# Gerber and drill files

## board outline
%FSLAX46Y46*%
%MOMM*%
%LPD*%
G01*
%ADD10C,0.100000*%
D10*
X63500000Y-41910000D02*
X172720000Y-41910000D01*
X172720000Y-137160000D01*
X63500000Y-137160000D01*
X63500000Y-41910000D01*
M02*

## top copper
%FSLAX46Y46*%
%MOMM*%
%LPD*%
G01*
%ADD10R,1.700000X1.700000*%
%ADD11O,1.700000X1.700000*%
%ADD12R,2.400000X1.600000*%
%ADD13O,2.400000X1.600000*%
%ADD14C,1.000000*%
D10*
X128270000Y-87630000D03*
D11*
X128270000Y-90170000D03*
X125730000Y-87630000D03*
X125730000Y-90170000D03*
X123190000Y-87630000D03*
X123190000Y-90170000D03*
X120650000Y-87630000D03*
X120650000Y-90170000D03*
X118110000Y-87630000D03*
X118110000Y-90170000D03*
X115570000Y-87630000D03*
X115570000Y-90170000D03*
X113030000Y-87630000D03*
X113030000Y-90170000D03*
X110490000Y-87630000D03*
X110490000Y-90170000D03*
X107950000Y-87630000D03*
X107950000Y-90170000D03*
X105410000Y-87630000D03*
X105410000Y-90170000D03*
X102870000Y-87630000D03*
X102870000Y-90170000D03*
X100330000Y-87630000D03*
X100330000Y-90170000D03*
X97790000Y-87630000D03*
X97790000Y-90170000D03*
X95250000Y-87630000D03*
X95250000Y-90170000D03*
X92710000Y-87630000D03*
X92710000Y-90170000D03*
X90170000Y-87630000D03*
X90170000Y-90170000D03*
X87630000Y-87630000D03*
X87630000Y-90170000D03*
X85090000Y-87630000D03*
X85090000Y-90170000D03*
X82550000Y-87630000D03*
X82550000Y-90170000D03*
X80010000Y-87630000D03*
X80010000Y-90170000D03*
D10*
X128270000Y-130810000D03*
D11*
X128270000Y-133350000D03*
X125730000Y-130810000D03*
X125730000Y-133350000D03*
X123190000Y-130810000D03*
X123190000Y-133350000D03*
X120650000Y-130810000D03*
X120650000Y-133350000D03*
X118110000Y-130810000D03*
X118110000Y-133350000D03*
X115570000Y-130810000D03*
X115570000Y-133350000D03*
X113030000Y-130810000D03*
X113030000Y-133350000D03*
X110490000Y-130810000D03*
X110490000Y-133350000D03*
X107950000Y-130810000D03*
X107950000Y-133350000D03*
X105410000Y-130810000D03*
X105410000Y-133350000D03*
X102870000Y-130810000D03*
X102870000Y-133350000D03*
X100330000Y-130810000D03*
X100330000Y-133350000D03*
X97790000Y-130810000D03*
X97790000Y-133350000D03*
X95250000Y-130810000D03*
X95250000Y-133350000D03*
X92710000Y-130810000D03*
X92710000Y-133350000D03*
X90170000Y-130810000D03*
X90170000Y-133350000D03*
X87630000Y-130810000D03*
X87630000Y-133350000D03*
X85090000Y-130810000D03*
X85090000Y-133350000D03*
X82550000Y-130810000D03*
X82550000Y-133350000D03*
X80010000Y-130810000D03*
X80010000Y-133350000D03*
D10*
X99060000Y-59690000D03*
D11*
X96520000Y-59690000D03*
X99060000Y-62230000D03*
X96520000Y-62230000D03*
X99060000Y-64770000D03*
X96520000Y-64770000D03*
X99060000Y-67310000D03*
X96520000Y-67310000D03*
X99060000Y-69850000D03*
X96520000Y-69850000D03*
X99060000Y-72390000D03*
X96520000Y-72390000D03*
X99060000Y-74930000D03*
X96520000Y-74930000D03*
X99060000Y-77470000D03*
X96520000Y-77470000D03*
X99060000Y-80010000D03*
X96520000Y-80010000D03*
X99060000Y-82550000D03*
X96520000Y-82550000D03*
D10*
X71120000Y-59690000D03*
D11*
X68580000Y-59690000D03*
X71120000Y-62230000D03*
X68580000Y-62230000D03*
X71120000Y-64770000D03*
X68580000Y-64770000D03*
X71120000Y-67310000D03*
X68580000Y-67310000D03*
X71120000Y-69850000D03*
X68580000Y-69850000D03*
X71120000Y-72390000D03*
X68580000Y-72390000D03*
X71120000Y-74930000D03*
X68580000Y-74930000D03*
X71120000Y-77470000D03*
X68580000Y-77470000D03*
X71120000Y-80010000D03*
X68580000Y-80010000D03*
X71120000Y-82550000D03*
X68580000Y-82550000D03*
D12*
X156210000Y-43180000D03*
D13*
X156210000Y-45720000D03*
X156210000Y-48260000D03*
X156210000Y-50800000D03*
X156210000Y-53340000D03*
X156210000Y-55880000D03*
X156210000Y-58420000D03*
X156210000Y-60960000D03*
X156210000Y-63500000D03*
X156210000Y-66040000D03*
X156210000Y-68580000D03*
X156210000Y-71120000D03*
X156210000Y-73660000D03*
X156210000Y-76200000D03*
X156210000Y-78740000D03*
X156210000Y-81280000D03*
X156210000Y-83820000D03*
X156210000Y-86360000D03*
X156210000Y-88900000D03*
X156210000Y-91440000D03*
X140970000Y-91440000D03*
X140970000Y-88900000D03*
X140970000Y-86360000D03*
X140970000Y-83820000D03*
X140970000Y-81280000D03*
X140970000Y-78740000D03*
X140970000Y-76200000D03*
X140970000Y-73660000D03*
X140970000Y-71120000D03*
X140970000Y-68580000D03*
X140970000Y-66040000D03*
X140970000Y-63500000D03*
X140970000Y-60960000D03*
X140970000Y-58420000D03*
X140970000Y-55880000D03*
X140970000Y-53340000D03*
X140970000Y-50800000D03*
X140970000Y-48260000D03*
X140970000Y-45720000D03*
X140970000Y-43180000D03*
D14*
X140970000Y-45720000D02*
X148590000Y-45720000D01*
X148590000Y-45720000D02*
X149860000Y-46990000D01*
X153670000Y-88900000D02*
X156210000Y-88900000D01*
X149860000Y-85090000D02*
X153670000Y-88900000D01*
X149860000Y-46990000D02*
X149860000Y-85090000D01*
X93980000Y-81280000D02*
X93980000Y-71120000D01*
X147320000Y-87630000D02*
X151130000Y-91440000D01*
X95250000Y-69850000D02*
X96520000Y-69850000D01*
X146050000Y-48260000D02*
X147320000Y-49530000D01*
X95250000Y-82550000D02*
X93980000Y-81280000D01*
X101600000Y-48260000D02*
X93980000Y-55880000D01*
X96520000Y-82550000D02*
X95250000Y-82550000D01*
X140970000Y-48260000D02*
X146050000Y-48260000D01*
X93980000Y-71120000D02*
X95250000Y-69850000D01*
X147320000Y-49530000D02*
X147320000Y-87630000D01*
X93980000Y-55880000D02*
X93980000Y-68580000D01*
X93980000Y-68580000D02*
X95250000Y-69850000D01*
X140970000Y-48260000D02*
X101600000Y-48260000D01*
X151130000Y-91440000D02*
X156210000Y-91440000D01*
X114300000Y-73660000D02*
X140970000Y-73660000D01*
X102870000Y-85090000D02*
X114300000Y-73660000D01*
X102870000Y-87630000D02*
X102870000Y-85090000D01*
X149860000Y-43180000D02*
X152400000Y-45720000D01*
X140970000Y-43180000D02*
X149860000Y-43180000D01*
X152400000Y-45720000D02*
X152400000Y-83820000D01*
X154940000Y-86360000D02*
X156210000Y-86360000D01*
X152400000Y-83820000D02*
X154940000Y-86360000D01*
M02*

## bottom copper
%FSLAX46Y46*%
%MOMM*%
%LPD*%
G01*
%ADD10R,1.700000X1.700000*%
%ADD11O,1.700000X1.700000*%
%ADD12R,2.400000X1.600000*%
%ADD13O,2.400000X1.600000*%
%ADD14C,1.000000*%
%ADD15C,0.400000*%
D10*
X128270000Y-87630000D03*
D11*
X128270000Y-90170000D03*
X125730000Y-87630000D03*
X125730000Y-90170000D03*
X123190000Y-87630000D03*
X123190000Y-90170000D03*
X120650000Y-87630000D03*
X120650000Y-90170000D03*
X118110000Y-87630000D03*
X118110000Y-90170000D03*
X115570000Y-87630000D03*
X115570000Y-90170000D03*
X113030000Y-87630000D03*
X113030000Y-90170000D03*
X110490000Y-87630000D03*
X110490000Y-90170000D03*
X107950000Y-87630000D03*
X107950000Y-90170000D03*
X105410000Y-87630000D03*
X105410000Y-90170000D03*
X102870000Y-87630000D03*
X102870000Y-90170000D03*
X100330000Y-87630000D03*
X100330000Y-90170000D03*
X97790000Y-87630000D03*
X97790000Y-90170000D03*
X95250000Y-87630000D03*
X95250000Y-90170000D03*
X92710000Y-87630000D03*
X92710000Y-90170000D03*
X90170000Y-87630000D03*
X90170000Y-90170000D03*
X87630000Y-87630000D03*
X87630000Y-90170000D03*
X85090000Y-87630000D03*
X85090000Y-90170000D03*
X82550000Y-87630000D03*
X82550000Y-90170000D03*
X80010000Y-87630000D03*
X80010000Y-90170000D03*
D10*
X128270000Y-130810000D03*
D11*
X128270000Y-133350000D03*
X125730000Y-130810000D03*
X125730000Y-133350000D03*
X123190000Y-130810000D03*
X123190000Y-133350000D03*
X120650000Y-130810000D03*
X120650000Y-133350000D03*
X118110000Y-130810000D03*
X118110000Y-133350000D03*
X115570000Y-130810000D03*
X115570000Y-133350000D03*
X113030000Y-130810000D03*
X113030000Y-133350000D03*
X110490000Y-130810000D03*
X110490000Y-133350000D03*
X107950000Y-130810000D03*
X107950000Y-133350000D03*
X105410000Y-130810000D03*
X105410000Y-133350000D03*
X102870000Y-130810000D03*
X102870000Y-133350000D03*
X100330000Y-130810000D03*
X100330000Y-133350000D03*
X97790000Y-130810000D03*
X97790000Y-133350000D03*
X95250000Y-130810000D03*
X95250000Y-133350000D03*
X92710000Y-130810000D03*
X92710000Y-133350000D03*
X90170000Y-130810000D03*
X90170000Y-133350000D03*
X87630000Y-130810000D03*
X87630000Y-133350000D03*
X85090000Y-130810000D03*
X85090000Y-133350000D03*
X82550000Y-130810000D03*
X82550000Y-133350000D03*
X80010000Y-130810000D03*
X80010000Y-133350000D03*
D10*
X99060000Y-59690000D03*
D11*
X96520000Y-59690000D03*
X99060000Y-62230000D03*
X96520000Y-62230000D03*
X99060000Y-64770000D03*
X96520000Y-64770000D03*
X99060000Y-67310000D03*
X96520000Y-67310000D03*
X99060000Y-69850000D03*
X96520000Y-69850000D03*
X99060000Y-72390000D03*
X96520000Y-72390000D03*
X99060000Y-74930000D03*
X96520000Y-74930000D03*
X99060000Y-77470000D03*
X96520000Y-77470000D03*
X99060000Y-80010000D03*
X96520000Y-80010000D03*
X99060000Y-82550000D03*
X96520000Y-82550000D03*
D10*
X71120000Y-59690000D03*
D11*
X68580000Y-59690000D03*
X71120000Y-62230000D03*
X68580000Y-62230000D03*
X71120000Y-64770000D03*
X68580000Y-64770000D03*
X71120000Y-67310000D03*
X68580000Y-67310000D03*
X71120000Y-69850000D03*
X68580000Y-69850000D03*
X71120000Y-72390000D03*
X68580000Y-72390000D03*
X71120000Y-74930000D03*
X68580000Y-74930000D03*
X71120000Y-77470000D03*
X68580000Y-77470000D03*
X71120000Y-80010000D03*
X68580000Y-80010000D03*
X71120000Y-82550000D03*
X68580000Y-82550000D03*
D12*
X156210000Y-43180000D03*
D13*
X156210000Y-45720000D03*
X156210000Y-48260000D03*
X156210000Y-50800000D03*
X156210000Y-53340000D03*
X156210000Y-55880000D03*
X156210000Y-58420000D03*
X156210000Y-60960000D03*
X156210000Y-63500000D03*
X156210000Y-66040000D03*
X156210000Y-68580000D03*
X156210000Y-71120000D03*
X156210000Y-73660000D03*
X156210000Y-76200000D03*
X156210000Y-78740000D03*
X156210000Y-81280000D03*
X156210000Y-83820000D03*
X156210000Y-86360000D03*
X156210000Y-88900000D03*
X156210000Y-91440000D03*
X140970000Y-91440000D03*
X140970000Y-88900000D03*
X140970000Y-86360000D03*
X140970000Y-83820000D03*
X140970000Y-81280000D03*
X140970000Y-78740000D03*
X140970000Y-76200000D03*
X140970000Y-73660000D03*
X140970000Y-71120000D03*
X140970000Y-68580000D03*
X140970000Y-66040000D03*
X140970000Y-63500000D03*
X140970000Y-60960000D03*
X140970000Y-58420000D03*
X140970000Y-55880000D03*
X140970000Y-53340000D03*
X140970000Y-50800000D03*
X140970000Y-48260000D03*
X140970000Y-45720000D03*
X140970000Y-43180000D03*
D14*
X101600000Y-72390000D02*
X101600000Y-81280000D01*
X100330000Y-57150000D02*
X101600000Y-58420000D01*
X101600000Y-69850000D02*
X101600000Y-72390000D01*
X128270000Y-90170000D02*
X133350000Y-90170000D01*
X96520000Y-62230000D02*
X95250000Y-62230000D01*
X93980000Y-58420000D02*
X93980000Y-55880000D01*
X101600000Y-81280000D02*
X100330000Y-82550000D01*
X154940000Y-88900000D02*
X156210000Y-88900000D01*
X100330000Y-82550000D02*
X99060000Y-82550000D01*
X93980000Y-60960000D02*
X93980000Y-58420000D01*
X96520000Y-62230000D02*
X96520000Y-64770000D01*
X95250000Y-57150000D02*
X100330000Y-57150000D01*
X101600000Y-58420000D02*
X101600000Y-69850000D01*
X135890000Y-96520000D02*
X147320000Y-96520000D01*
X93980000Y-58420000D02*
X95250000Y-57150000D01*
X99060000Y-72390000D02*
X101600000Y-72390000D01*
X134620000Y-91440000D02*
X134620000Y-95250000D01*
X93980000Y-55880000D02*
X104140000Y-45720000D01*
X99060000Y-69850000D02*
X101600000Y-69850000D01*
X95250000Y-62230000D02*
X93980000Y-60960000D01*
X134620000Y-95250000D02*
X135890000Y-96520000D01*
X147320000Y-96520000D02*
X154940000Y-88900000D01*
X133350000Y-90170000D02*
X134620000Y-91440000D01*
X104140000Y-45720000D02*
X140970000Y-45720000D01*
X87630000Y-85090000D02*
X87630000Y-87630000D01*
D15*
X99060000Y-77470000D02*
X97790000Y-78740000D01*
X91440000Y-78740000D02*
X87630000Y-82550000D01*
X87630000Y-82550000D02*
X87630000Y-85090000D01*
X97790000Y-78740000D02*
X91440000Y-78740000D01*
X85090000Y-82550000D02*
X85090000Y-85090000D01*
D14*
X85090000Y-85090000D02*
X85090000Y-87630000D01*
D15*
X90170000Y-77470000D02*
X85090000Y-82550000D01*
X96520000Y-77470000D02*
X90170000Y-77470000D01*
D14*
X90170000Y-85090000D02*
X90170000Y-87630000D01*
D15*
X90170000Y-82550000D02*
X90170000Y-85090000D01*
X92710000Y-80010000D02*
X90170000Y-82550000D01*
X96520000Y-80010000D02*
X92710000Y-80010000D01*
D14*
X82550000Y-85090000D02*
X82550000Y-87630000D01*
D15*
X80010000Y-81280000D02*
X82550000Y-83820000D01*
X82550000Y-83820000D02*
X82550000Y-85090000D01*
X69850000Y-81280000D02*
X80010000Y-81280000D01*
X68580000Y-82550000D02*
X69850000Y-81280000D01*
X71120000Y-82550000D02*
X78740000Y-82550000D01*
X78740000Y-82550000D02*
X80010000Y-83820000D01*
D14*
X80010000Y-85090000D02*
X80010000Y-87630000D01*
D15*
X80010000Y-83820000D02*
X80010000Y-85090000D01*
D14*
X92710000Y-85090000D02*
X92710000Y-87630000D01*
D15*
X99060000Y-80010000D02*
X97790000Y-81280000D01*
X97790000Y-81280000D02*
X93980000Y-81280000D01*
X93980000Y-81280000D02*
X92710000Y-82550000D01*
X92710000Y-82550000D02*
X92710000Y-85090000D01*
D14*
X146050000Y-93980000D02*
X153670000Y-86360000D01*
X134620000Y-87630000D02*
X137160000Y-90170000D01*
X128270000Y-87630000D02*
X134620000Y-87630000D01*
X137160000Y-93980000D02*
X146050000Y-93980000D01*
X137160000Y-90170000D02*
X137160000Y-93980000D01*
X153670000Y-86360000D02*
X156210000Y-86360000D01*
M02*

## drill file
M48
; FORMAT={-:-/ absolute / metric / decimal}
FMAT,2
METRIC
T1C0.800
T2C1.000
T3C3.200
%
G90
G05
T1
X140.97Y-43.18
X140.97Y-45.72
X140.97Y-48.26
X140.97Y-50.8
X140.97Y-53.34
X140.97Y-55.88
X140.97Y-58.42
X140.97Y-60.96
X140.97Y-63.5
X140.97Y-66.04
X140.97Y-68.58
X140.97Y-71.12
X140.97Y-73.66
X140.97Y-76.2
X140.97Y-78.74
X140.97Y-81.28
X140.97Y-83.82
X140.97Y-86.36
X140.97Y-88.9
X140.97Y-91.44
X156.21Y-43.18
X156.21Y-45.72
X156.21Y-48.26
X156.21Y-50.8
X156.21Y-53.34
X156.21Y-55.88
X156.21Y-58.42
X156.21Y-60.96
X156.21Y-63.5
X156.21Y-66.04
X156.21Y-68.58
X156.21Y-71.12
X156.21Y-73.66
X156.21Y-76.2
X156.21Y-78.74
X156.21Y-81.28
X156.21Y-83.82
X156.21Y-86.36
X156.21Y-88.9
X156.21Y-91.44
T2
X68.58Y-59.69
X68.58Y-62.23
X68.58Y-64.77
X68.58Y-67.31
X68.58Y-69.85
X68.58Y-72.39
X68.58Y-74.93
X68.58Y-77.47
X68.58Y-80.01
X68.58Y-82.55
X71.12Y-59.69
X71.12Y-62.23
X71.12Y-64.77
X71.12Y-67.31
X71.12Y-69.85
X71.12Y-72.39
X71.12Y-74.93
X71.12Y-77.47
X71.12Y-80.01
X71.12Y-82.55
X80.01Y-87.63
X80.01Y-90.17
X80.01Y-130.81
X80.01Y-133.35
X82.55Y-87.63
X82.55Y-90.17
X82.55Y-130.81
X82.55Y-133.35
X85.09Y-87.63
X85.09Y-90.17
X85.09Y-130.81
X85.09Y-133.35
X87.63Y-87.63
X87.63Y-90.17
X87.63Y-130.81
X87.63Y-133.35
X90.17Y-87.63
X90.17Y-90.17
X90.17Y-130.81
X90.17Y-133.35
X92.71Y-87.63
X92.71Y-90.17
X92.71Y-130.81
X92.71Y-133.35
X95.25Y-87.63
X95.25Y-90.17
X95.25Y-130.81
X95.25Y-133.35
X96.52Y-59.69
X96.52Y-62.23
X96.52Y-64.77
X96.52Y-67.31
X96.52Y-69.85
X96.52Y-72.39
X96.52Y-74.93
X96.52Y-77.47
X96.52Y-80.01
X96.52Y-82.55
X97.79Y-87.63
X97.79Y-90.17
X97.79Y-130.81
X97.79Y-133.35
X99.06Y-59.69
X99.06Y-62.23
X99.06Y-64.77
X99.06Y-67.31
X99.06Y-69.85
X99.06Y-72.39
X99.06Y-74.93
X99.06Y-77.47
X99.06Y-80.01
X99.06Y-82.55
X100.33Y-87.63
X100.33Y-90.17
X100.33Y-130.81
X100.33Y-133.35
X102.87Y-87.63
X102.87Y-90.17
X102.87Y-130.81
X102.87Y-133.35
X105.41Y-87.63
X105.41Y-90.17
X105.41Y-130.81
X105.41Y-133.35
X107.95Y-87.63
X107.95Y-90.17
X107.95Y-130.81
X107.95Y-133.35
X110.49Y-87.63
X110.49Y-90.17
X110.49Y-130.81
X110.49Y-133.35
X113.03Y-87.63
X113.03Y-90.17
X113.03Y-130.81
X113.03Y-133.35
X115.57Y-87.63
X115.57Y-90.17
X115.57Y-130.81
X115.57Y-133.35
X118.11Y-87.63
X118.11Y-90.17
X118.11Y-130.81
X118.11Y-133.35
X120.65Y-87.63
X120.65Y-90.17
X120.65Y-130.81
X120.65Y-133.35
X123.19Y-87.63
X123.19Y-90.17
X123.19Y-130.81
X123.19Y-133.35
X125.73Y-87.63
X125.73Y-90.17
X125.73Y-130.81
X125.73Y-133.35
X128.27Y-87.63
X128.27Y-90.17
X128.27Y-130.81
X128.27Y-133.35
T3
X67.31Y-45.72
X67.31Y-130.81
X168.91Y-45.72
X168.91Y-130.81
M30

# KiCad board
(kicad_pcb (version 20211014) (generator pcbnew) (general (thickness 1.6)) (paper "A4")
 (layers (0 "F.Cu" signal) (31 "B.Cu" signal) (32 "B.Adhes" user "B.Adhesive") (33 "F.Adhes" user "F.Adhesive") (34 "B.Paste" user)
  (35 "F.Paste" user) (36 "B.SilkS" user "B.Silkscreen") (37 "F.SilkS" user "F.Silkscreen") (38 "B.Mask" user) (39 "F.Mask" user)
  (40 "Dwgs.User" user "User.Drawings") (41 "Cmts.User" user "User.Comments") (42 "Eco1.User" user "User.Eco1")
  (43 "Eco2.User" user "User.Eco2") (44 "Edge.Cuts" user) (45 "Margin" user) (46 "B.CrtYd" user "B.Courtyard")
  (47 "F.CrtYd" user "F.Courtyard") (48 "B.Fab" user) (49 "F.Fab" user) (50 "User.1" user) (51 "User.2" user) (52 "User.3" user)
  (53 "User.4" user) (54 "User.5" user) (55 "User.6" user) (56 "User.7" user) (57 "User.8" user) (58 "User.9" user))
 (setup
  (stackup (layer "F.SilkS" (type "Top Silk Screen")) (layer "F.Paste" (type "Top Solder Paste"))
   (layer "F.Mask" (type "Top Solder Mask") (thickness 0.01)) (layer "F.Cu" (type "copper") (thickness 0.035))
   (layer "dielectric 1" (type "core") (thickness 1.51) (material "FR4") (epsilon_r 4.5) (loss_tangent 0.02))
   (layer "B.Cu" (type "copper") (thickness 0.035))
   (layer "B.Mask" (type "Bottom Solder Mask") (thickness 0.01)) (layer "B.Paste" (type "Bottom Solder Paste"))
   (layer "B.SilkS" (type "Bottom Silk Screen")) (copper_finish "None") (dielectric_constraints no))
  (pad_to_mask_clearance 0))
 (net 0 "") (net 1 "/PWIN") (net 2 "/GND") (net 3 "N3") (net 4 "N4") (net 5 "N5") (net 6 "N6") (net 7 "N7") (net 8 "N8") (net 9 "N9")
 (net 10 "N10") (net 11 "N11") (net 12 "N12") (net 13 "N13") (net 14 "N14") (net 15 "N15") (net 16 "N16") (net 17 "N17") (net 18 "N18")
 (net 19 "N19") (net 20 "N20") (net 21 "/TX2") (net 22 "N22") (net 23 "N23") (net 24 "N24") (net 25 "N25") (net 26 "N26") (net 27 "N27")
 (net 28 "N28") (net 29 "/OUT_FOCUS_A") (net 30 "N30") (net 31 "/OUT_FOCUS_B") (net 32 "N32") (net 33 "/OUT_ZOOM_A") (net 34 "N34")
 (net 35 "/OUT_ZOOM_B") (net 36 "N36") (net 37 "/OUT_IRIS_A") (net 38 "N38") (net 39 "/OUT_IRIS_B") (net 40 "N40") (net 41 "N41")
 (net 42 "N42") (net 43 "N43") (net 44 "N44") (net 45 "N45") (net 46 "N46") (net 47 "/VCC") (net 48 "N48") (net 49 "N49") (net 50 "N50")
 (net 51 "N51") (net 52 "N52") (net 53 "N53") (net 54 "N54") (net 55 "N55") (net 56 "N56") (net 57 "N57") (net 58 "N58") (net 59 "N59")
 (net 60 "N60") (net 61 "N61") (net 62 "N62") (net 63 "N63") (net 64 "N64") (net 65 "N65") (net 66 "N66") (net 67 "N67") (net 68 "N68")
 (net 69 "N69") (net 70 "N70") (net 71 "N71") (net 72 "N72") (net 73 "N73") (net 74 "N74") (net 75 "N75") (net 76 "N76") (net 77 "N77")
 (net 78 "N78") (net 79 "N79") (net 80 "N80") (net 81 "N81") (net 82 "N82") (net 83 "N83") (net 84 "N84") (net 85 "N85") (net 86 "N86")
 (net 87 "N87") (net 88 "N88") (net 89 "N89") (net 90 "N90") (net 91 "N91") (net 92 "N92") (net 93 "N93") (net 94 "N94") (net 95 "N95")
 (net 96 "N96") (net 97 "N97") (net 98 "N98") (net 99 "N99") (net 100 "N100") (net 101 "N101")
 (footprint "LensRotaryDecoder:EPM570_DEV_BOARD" (layer "F.Cu") (at 102.87 110.49 -90)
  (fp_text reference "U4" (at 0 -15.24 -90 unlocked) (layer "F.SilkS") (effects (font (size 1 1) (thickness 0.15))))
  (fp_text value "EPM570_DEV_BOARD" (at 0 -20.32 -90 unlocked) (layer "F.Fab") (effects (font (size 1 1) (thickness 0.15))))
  (pad "1" thru_hole rect (at -22.86 -25.4 270) (size 1.7 1.7) (drill 1) (layers *.Cu *.Mask) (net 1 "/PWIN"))
  (pad "2" thru_hole oval (at -20.32 -25.4 270) (size 1.7 1.7) (drill 1) (layers *.Cu *.Mask) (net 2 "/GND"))
  (pad "3" thru_hole oval (at -22.86 -22.86 270) (size 1.7 1.7) (drill 1) (layers *.Cu *.Mask) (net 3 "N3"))
  (pad "4" thru_hole oval (at -20.32 -22.86 270) (size 1.7 1.7) (drill 1) (layers *.Cu *.Mask) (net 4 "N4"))
  (pad "5" thru_hole oval (at -22.86 -20.32 270) (size 1.7 1.7) (drill 1) (layers *.Cu *.Mask) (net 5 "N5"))
  (pad "6" thru_hole oval (at -20.32 -20.32 270) (size 1.7 1.7) (drill 1) (layers *.Cu *.Mask) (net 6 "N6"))
  (pad "7" thru_hole oval (at -22.86 -17.78 270) (size 1.7 1.7) (drill 1) (layers *.Cu *.Mask) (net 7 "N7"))
  (pad "8" thru_hole oval (at -20.32 -17.78 270) (size 1.7 1.7) (drill 1) (layers *.Cu *.Mask) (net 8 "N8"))
  (pad "9" thru_hole oval (at -22.86 -15.24 270) (size 1.7 1.7) (drill 1) (layers *.Cu *.Mask) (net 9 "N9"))
  (pad "10" thru_hole oval (at -20.32 -15.24 270) (size 1.7 1.7) (drill 1) (layers *.Cu *.Mask) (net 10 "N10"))
  (pad "11" thru_hole oval (at -22.86 -12.7 270) (size 1.7 1.7) (drill 1) (layers *.Cu *.Mask) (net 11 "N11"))
  (pad "12" thru_hole oval (at -20.32 -12.7 270) (size 1.7 1.7) (drill 1) (layers *.Cu *.Mask) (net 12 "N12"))
  (pad "13" thru_hole oval (at -22.86 -10.16 270) (size 1.7 1.7) (drill 1) (layers *.Cu *.Mask) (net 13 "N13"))
  (pad "14" thru_hole oval (at -20.32 -10.16 270) (size 1.7 1.7) (drill 1) (layers *.Cu *.Mask) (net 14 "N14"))
  (pad "15" thru_hole oval (at -22.86 -7.62 270) (size 1.7 1.7) (drill 1) (layers *.Cu *.Mask) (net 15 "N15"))
  (pad "16" thru_hole oval (at -20.32 -7.62 270) (size 1.7 1.7) (drill 1) (layers *.Cu *.Mask) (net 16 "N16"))
  (pad "17" thru_hole oval (at -22.86 -5.08 270) (size 1.7 1.7) (drill 1) (layers *.Cu *.Mask) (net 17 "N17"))
  (pad "18" thru_hole oval (at -20.32 -5.08 270) (size 1.7 1.7) (drill 1) (layers *.Cu *.Mask) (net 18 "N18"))
  (pad "19" thru_hole oval (at -22.86 -2.54 270) (size 1.7 1.7) (drill 1) (layers *.Cu *.Mask) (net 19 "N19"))
  (pad "20" thru_hole oval (at -20.32 -2.54 270) (size 1.7 1.7) (drill 1) (layers *.Cu *.Mask) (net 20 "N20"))
  (pad "21" thru_hole oval (at -22.86 0 270) (size 1.7 1.7) (drill 1) (layers *.Cu *.Mask) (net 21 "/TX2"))
  (pad "22" thru_hole oval (at -20.32 0 270) (size 1.7 1.7) (drill 1) (layers *.Cu *.Mask) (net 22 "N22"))
  (pad "23" thru_hole oval (at -22.86 2.54 270) (size 1.7 1.7) (drill 1) (layers *.Cu *.Mask) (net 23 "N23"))
  (pad "24" thru_hole oval (at -20.32 2.54 270) (size 1.7 1.7) (drill 1) (layers *.Cu *.Mask) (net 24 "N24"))
  (pad "25" thru_hole oval (at -22.86 5.08 270) (size 1.7 1.7) (drill 1) (layers *.Cu *.Mask) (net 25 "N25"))
  (pad "26" thru_hole oval (at -20.32 5.08 270) (size 1.7 1.7) (drill 1) (layers *.Cu *.Mask) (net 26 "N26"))
  (pad "27" thru_hole oval (at -22.86 7.62 270) (size 1.7 1.7) (drill 1) (layers *.Cu *.Mask) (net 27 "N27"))
  (pad "28" thru_hole oval (at -20.32 7.62 270) (size 1.7 1.7) (drill 1) (layers *.Cu *.Mask) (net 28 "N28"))
  (pad "29" thru_hole oval (at -22.86 10.16 270) (size 1.7 1.7) (drill 1) (layers *.Cu *.Mask) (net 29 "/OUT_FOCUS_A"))
  (pad "30" thru_hole oval (at -20.32 10.16 270) (size 1.7 1.7) (drill 1) (layers *.Cu *.Mask) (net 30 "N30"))
  (pad "31" thru_hole oval (at -22.86 12.7 270) (size 1.7 1.7) (drill 1) (layers *.Cu *.Mask) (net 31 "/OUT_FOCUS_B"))
  (pad "32" thru_hole oval (at -20.32 12.7 270) (size 1.7 1.7) (drill 1) (layers *.Cu *.Mask) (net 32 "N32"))
  (pad "33" thru_hole oval (at -22.86 15.24 270) (size 1.7 1.7) (drill 1) (layers *.Cu *.Mask) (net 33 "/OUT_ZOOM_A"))
  (pad "34" thru_hole oval (at -20.32 15.24 270) (size 1.7 1.7) (drill 1) (layers *.Cu *.Mask) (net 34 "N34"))
  (pad "35" thru_hole oval (at -22.86 17.78 270) (size 1.7 1.7) (drill 1) (layers *.Cu *.Mask) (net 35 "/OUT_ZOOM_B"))
  (pad "36" thru_hole oval (at -20.32 17.78 270) (size 1.7 1.7) (drill 1) (layers *.Cu *.Mask) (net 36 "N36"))
  (pad "37" thru_hole oval (at -22.86 20.32 270) (size 1.7 1.7) (drill 1) (layers *.Cu *.Mask) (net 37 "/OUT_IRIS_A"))
  (pad "38" thru_hole oval (at -20.32 20.32 270) (size 1.7 1.7) (drill 1) (layers *.Cu *.Mask) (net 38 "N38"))
  (pad "39" thru_hole oval (at -22.86 22.86 270) (size 1.7 1.7) (drill 1) (layers *.Cu *.Mask) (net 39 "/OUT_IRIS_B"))
  (pad "40" thru_hole oval (at -20.32 22.86 270) (size 1.7 1.7) (drill 1) (layers *.Cu *.Mask) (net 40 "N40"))
  (pad "41" thru_hole rect (at 20.32 -25.4 270) (size 1.7 1.7) (drill 1) (layers *.Cu *.Mask))
  (pad "42" thru_hole oval (at 22.86 -25.4 270) (size 1.7 1.7) (drill 1) (layers *.Cu *.Mask))
  (pad "43" thru_hole oval (at 20.32 -22.86 270) (size 1.7 1.7) (drill 1) (layers *.Cu *.Mask))
  (pad "44" thru_hole oval (at 22.86 -22.86 270) (size 1.7 1.7) (drill 1) (layers *.Cu *.Mask))
  (pad "45" thru_hole oval (at 20.32 -20.32 270) (size 1.7 1.7) (drill 1) (layers *.Cu *.Mask))
  (pad "46" thru_hole oval (at 22.86 -20.32 270) (size 1.7 1.7) (drill 1) (layers *.Cu *.Mask))
  (pad "47" thru_hole oval (at 20.32 -17.78 270) (size 1.7 1.7) (drill 1) (layers *.Cu *.Mask))
  (pad "48" thru_hole oval (at 22.86 -17.78 270) (size 1.7 1.7) (drill 1) (layers *.Cu *.Mask))
  (pad "49" thru_hole oval (at 20.32 -15.24 270) (size 1.7 1.7) (drill 1) (layers *.Cu *.Mask))
  (pad "50" thru_hole oval (at 22.86 -15.24 270) (size 1.7 1.7) (drill 1) (layers *.Cu *.Mask))
  (pad "51" thru_hole oval (at 20.32 -12.7 270) (size 1.7 1.7) (drill 1) (layers *.Cu *.Mask))
  (pad "52" thru_hole oval (at 22.86 -12.7 270) (size 1.7 1.7) (drill 1) (layers *.Cu *.Mask))
  (pad "53" thru_hole oval (at 20.32 -10.16 270) (size 1.7 1.7) (drill 1) (layers *.Cu *.Mask))
  (pad "54" thru_hole oval (at 22.86 -10.16 270) (size 1.7 1.7) (drill 1) (layers *.Cu *.Mask))
  (pad "55" thru_hole oval (at 20.32 -7.62 270) (size 1.7 1.7) (drill 1) (layers *.Cu *.Mask))
  (pad "56" thru_hole oval (at 22.86 -7.62 270) (size 1.7 1.7) (drill 1) (layers *.Cu *.Mask))
  (pad "57" thru_hole oval (at 20.32 -5.08 270) (size 1.7 1.7) (drill 1) (layers *.Cu *.Mask))
  (pad "58" thru_hole oval (at 22.86 -5.08 270) (size 1.7 1.7) (drill 1) (layers *.Cu *.Mask))
  (pad "59" thru_hole oval (at 20.32 -2.54 270) (size 1.7 1.7) (drill 1) (layers *.Cu *.Mask))
  (pad "60" thru_hole oval (at 22.86 -2.54 270) (size 1.7 1.7) (drill 1) (layers *.Cu *.Mask))
  (pad "61" thru_hole oval (at 20.32 0 270) (size 1.7 1.7) (drill 1) (layers *.Cu *.Mask))
  (pad "62" thru_hole oval (at 22.86 0 270) (size 1.7 1.7) (drill 1) (layers *.Cu *.Mask))
  (pad "63" thru_hole oval (at 20.32 2.54 270) (size 1.7 1.7) (drill 1) (layers *.Cu *.Mask))
  (pad "64" thru_hole oval (at 22.86 2.54 270) (size 1.7 1.7) (drill 1) (layers *.Cu *.Mask))
  (pad "65" thru_hole oval (at 20.32 5.08 270) (size 1.7 1.7) (drill 1) (layers *.Cu *.Mask))
  (pad "66" thru_hole oval (at 22.86 5.08 270) (size 1.7 1.7) (drill 1) (layers *.Cu *.Mask))
  (pad "67" thru_hole oval (at 20.32 7.62 270) (size 1.7 1.7) (drill 1) (layers *.Cu *.Mask))
  (pad "68" thru_hole oval (at 22.86 7.62 270) (size 1.7 1.7) (drill 1) (layers *.Cu *.Mask))
  (pad "69" thru_hole oval (at 20.32 10.16 270) (size 1.7 1.7) (drill 1) (layers *.Cu *.Mask))
  (pad "70" thru_hole oval (at 22.86 10.16 270) (size 1.7 1.7) (drill 1) (layers *.Cu *.Mask))
  (pad "71" thru_hole oval (at 20.32 12.7 270) (size 1.7 1.7) (drill 1) (layers *.Cu *.Mask))
  (pad "72" thru_hole oval (at 22.86 12.7 270) (size 1.7 1.7) (drill 1) (layers *.Cu *.Mask))
  (pad "73" thru_hole oval (at 20.32 15.24 270) (size 1.7 1.7) (drill 1) (layers *.Cu *.Mask))
  (pad "74" thru_hole oval (at 22.86 15.24 270) (size 1.7 1.7) (drill 1) (layers *.Cu *.Mask))
  (pad "75" thru_hole oval (at 20.32 17.78 270) (size 1.7 1.7) (drill 1) (layers *.Cu *.Mask))
  (pad "76" thru_hole oval (at 22.86 17.78 270) (size 1.7 1.7) (drill 1) (layers *.Cu *.Mask))
  (pad "77" thru_hole oval (at 20.32 20.32 270) (size 1.7 1.7) (drill 1) (layers *.Cu *.Mask))
  (pad "78" thru_hole oval (at 22.86 20.32 270) (size 1.7 1.7) (drill 1) (layers *.Cu *.Mask))
  (pad "79" thru_hole oval (at 20.32 22.86 270) (size 1.7 1.7) (drill 1) (layers *.Cu *.Mask))
  (pad "80" thru_hole oval (at 22.86 22.86 270) (size 1.7 1.7) (drill 1) (layers *.Cu *.Mask)))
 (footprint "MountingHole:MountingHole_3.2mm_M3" (layer "F.Cu") (at 67.31 130.81)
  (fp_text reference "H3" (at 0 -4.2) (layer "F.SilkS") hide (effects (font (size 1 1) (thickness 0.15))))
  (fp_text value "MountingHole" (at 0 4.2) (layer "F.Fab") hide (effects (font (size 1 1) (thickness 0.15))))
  (pad "" np_thru_hole circle locked (at 0 0) (size 3.2 3.2) (drill 3.2) (layers *.Cu *.Mask)))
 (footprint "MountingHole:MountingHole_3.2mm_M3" (layer "F.Cu") (at 168.91 130.81)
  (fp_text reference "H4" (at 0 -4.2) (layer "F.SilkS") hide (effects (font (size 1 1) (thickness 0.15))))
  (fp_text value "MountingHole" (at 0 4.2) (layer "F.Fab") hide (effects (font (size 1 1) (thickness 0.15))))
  (pad "" np_thru_hole circle locked (at 0 0) (size 3.2 3.2) (drill 3.2) (layers *.Cu *.Mask)))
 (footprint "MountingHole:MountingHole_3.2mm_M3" (layer "F.Cu") (at 168.91 45.72)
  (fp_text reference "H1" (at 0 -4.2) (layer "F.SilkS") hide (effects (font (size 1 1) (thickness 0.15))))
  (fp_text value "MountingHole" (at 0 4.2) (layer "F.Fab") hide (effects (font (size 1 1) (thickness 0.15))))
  (pad "" np_thru_hole circle locked (at 0 0) (size 3.2 3.2) (drill 3.2) (layers *.Cu *.Mask)))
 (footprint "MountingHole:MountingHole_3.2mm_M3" (layer "F.Cu") (at 67.31 45.72)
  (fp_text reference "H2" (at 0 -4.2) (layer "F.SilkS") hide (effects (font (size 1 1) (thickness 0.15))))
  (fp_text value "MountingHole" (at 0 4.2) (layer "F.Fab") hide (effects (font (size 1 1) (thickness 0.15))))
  (pad "" np_thru_hole circle locked (at 0 0) (size 3.2 3.2) (drill 3.2) (layers *.Cu *.Mask)))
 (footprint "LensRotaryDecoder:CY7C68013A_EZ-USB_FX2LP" (layer "B.Cu") (at 87.09 71.115 180)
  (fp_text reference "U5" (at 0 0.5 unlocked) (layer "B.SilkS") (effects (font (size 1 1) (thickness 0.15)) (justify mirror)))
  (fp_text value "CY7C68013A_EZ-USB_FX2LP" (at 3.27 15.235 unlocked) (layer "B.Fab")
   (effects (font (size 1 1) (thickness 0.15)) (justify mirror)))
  (pad "1" thru_hole rect (at -11.97 11.425 180) (size 1.7 1.7) (drill 1) (layers *.Cu *.Mask) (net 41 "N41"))
  (pad "2" thru_hole oval (at -9.43 11.425 180) (size 1.7 1.7) (drill 1) (layers *.Cu *.Mask) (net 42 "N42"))
  (pad "3" thru_hole oval (at -11.97 8.885 180) (size 1.7 1.7) (drill 1) (layers *.Cu *.Mask) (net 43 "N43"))
  (pad "4" thru_hole oval (at -9.43 8.885 180) (size 1.7 1.7) (drill 1) (layers *.Cu *.Mask) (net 2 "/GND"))
  (pad "5" thru_hole oval (at -11.97 6.345 180) (size 1.7 1.7) (drill 1) (layers *.Cu *.Mask) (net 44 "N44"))
  (pad "6" thru_hole oval (at -9.43 6.345 180) (size 1.7 1.7) (drill 1) (layers *.Cu *.Mask) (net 2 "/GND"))
  (pad "7" thru_hole oval (at -11.97 3.805 180) (size 1.7 1.7) (drill 1) (layers *.Cu *.Mask) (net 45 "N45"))
  (pad "8" thru_hole oval (at -9.43 3.805 180) (size 1.7 1.7) (drill 1) (layers *.Cu *.Mask) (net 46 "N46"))
  (pad "9" thru_hole oval (at -11.97 1.265 180) (size 1.7 1.7) (drill 1) (layers *.Cu *.Mask) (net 2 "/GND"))
  (pad "10" thru_hole oval (at -9.43 1.265 180) (size 1.7 1.7) (drill 1) (layers *.Cu *.Mask) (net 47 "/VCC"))
  (pad "11" thru_hole oval (at -11.97 -1.275 180) (size 1.7 1.7) (drill 1) (layers *.Cu *.Mask) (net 2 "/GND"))
  (pad "12" thru_hole oval (at -9.43 -1.275 180) (size 1.7 1.7) (drill 1) (layers *.Cu *.Mask) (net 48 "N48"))
  (pad "13" thru_hole oval (at -11.97 -3.815 180) (size 1.7 1.7) (drill 1) (layers *.Cu *.Mask) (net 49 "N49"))
  (pad "14" thru_hole oval (at -9.43 -3.815 180) (size 1.7 1.7) (drill 1) (layers *.Cu *.Mask) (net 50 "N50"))
  (pad "15" thru_hole oval (at -11.97 -6.355 180) (size 1.7 1.7) (drill 1) (layers *.Cu *.Mask) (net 33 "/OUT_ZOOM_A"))
  (pad "16" thru_hole oval (at -9.43 -6.355 180) (size 1.7 1.7) (drill 1) (layers *.Cu *.Mask) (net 35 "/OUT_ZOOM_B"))
  (pad "17" thru_hole oval (at -11.97 -8.895 180) (size 1.7 1.7) (drill 1) (layers *.Cu *.Mask) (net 29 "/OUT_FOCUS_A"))
  (pad "18" thru_hole oval (at -9.43 -8.895 180) (size 1.7 1.7) (drill 1) (layers *.Cu *.Mask) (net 31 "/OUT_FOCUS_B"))
  (pad "19" thru_hole oval (at -11.97 -11.435 180) (size 1.7 1.7) (drill 1) (layers *.Cu *.Mask) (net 2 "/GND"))
  (pad "20" thru_hole oval (at -9.43 -11.435 180) (size 1.7 1.7) (drill 1) (layers *.Cu *.Mask) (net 47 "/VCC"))
  (pad "21" thru_hole rect (at 15.97 11.425 180) (size 1.7 1.7) (drill 1) (layers *.Cu *.Mask) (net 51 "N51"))
  (pad "22" thru_hole oval (at 18.51 11.425 180) (size 1.7 1.7) (drill 1) (layers *.Cu *.Mask) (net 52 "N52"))
  (pad "23" thru_hole oval (at 15.97 8.885 180) (size 1.7 1.7) (drill 1) (layers *.Cu *.Mask) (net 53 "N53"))
  (pad "24" thru_hole oval (at 18.51 8.885 180) (size 1.7 1.7) (drill 1) (layers *.Cu *.Mask) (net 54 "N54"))
  (pad "25" thru_hole oval (at 15.97 6.345 180) (size 1.7 1.7) (drill 1) (layers *.Cu *.Mask) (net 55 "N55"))
  (pad "26" thru_hole oval (at 18.51 6.345 180) (size 1.7 1.7) (drill 1) (layers *.Cu *.Mask) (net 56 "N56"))
  (pad "27" thru_hole oval (at 15.97 3.805 180) (size 1.7 1.7) (drill 1) (layers *.Cu *.Mask) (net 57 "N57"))
  (pad "28" thru_hole oval (at 18.51 3.805 180) (size 1.7 1.7) (drill 1) (layers *.Cu *.Mask) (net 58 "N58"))
  (pad "29" thru_hole oval (at 15.97 1.265 180) (size 1.7 1.7) (drill 1) (layers *.Cu *.Mask) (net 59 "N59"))
  (pad "30" thru_hole oval (at 18.51 1.265 180) (size 1.7 1.7) (drill 1) (layers *.Cu *.Mask) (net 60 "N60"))
  (pad "31" thru_hole oval (at 15.97 -1.275 180) (size 1.7 1.7) (drill 1) (layers *.Cu *.Mask) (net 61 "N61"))
  (pad "32" thru_hole oval (at 18.51 -1.275 180) (size 1.7 1.7) (drill 1) (layers *.Cu *.Mask) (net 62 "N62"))
  (pad "33" thru_hole oval (at 15.97 -3.815 180) (size 1.7 1.7) (drill 1) (layers *.Cu *.Mask) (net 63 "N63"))
  (pad "34" thru_hole oval (at 18.51 -3.815 180) (size 1.7 1.7) (drill 1) (layers *.Cu *.Mask) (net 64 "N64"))
  (pad "35" thru_hole oval (at 15.97 -6.355 180) (size 1.7 1.7) (drill 1) (layers *.Cu *.Mask) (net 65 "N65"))
  (pad "36" thru_hole oval (at 18.51 -6.355 180) (size 1.7 1.7) (drill 1) (layers *.Cu *.Mask) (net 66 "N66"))
  (pad "37" thru_hole oval (at 15.97 -8.895 180) (size 1.7 1.7) (drill 1) (layers *.Cu *.Mask) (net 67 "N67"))
  (pad "38" thru_hole oval (at 18.51 -8.895 180) (size 1.7 1.7) (drill 1) (layers *.Cu *.Mask) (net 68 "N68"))
  (pad "39" thru_hole oval (at 15.97 -11.435 180) (size 1.7 1.7) (drill 1) (layers *.Cu *.Mask) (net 39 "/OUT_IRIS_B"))
  (pad "40" thru_hole oval (at 18.51 -11.435 180) (size 1.7 1.7) (drill 1) (layers *.Cu *.Mask) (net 37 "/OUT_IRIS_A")))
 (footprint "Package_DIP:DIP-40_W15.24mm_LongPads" (layer "B.Cu") (at 156.21 43.18 180)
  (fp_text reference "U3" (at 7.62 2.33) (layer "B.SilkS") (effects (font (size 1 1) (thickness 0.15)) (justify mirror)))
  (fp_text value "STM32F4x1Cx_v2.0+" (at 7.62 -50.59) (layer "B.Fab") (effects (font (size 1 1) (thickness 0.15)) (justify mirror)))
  (pad "1" thru_hole rect locked (at 0 0 180) (size 2.4 1.6) (drill 0.8) (layers *.Cu *.Mask) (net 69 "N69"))
  (pad "2" thru_hole oval locked (at 0 -2.54 180) (size 2.4 1.6) (drill 0.8) (layers *.Cu *.Mask) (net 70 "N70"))
  (pad "3" thru_hole oval locked (at 0 -5.08 180) (size 2.4 1.6) (drill 0.8) (layers *.Cu *.Mask) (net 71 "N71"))
  (pad "4" thru_hole oval locked (at 0 -7.62 180) (size 2.4 1.6) (drill 0.8) (layers *.Cu *.Mask) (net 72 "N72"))
  (pad "5" thru_hole oval locked (at 0 -10.16 180) (size 2.4 1.6) (drill 0.8) (layers *.Cu *.Mask) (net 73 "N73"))
  (pad "6" thru_hole oval locked (at 0 -12.7 180) (size 2.4 1.6) (drill 0.8) (layers *.Cu *.Mask) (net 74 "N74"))
  (pad "7" thru_hole oval locked (at 0 -15.24 180) (size 2.4 1.6) (drill 0.8) (layers *.Cu *.Mask) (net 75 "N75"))
  (pad "8" thru_hole oval locked (at 0 -17.78 180) (size 2.4 1.6) (drill 0.8) (layers *.Cu *.Mask) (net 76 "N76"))
  (pad "9" thru_hole oval locked (at 0 -20.32 180) (size 2.4 1.6) (drill 0.8) (layers *.Cu *.Mask) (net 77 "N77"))
  (pad "10" thru_hole oval locked (at 0 -22.86 180) (size 2.4 1.6) (drill 0.8) (layers *.Cu *.Mask) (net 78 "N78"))
  (pad "11" thru_hole oval locked (at 0 -25.4 180) (size 2.4 1.6) (drill 0.8) (layers *.Cu *.Mask) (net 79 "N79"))
  (pad "12" thru_hole oval locked (at 0 -27.94 180) (size 2.4 1.6) (drill 0.8) (layers *.Cu *.Mask) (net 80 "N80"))
  (pad "13" thru_hole oval locked (at 0 -30.48 180) (size 2.4 1.6) (drill 0.8) (layers *.Cu *.Mask) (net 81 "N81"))
  (pad "14" thru_hole oval locked (at 0 -33.02 180) (size 2.4 1.6) (drill 0.8) (layers *.Cu *.Mask) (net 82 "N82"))
  (pad "15" thru_hole oval locked (at 0 -35.56 180) (size 2.4 1.6) (drill 0.8) (layers *.Cu *.Mask) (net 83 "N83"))
  (pad "16" thru_hole oval locked (at 0 -38.1 180) (size 2.4 1.6) (drill 0.8) (layers *.Cu *.Mask) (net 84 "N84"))
  (pad "17" thru_hole oval locked (at 0 -40.64 180) (size 2.4 1.6) (drill 0.8) (layers *.Cu *.Mask) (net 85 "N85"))
  (pad "18" thru_hole oval locked (at 0 -43.18 180) (size 2.4 1.6) (drill 0.8) (layers *.Cu *.Mask) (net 1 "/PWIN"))
  (pad "19" thru_hole oval locked (at 0 -45.72 180) (size 2.4 1.6) (drill 0.8) (layers *.Cu *.Mask) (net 2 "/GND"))
  (pad "20" thru_hole oval locked (at 0 -48.26 180) (size 2.4 1.6) (drill 0.8) (layers *.Cu *.Mask) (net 47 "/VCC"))
  (pad "21" thru_hole oval locked (at 15.24 -48.26 180) (size 2.4 1.6) (drill 0.8) (layers *.Cu *.Mask) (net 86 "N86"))
  (pad "22" thru_hole oval locked (at 15.24 -45.72 180) (size 2.4 1.6) (drill 0.8) (layers *.Cu *.Mask) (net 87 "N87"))
  (pad "23" thru_hole oval locked (at 15.24 -43.18 180) (size 2.4 1.6) (drill 0.8) (layers *.Cu *.Mask) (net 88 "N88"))
  (pad "24" thru_hole oval locked (at 15.24 -40.64 180) (size 2.4 1.6) (drill 0.8) (layers *.Cu *.Mask) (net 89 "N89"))
  (pad "25" thru_hole oval locked (at 15.24 -38.1 180) (size 2.4 1.6) (drill 0.8) (layers *.Cu *.Mask) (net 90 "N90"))
  (pad "26" thru_hole oval locked (at 15.24 -35.56 180) (size 2.4 1.6) (drill 0.8) (layers *.Cu *.Mask) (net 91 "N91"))
  (pad "27" thru_hole oval locked (at 15.24 -33.02 180) (size 2.4 1.6) (drill 0.8) (layers *.Cu *.Mask) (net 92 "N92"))
  (pad "28" thru_hole oval locked (at 15.24 -30.48 180) (size 2.4 1.6) (drill 0.8) (layers *.Cu *.Mask) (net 21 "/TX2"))
  (pad "29" thru_hole oval locked (at 15.24 -27.94 180) (size 2.4 1.6) (drill 0.8) (layers *.Cu *.Mask) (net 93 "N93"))
  (pad "30" thru_hole oval locked (at 15.24 -25.4 180) (size 2.4 1.6) (drill 0.8) (layers *.Cu *.Mask) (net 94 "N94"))
  (pad "31" thru_hole oval locked (at 15.24 -22.86 180) (size 2.4 1.6) (drill 0.8) (layers *.Cu *.Mask) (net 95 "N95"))
  (pad "32" thru_hole oval locked (at 15.24 -20.32 180) (size 2.4 1.6) (drill 0.8) (layers *.Cu *.Mask) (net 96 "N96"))
  (pad "33" thru_hole oval locked (at 15.24 -17.78 180) (size 2.4 1.6) (drill 0.8) (layers *.Cu *.Mask) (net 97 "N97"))
  (pad "34" thru_hole oval locked (at 15.24 -15.24 180) (size 2.4 1.6) (drill 0.8) (layers *.Cu *.Mask) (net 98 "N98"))
  (pad "35" thru_hole oval locked (at 15.24 -12.7 180) (size 2.4 1.6) (drill 0.8) (layers *.Cu *.Mask) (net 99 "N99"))
  (pad "36" thru_hole oval locked (at 15.24 -10.16 180) (size 2.4 1.6) (drill 0.8) (layers *.Cu *.Mask) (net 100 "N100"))
  (pad "37" thru_hole oval locked (at 15.24 -7.62 180) (size 2.4 1.6) (drill 0.8) (layers *.Cu *.Mask) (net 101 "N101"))
  (pad "38" thru_hole oval locked (at 15.24 -5.08 180) (size 2.4 1.6) (drill 0.8) (layers *.Cu *.Mask) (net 47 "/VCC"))
  (pad "39" thru_hole oval locked (at 15.24 -2.54 180) (size 2.4 1.6) (drill 0.8) (layers *.Cu *.Mask) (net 2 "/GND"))
  (pad "40" thru_hole oval locked (at 15.24 0 180) (size 2.4 1.6) (drill 0.8) (layers *.Cu *.Mask) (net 1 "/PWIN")))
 (gr_rect (start 63.5 41.91) (end 172.72 137.16) (layer "Edge.Cuts") (width 0.1) (fill none))
 (segment (start 140.97 45.72) (end 148.59 45.72) (width 1) (layer "F.Cu") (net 2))
 (segment (start 148.59 45.72) (end 149.86 46.99) (width 1) (layer "F.Cu") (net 2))
 (segment (start 153.67 88.9) (end 156.21 88.9) (width 1) (layer "F.Cu") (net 2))
 (segment (start 149.86 85.09) (end 153.67 88.9) (width 1) (layer "F.Cu") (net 2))
 (segment (start 149.86 46.99) (end 149.86 85.09) (width 1) (layer "F.Cu") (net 2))
 (segment (start 101.6 72.39) (end 101.6 81.28) (width 1) (layer "B.Cu") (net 2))
 (segment (start 100.33 57.15) (end 101.6 58.42) (width 1) (layer "B.Cu") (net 2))
 (segment (start 101.6 69.85) (end 101.6 72.39) (width 1) (layer "B.Cu") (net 2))
 (segment (start 128.27 90.17) (end 133.35 90.17) (width 1) (layer "B.Cu") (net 2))
 (segment (start 96.52 62.23) (end 95.25 62.23) (width 1) (layer "B.Cu") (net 2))
 (segment (start 93.98 58.42) (end 93.98 55.88) (width 1) (layer "B.Cu") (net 2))
 (segment (start 101.6 81.28) (end 100.33 82.55) (width 1) (layer "B.Cu") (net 2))
 (segment (start 154.94 88.9) (end 156.21 88.9) (width 1) (layer "B.Cu") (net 2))
 (segment (start 100.33 82.55) (end 99.06 82.55) (width 1) (layer "B.Cu") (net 2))
 (segment (start 93.98 60.96) (end 93.98 58.42) (width 1) (layer "B.Cu") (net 2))
 (segment (start 96.52 62.23) (end 96.52 64.77) (width 1) (layer "B.Cu") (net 2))
 (segment (start 95.25 57.15) (end 100.33 57.15) (width 1) (layer "B.Cu") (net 2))
 (segment (start 101.6 58.42) (end 101.6 69.85) (width 1) (layer "B.Cu") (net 2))
 (segment (start 135.89 96.52) (end 147.32 96.52) (width 1) (layer "B.Cu") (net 2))
 (segment (start 93.98 58.42) (end 95.25 57.15) (width 1) (layer "B.Cu") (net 2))
 (segment (start 99.06 72.39) (end 101.6 72.39) (width 1) (layer "B.Cu") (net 2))
 (segment (start 134.62 91.44) (end 134.62 95.25) (width 1) (layer "B.Cu") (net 2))
 (segment (start 93.98 55.88) (end 104.14 45.72) (width 1) (layer "B.Cu") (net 2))
 (segment (start 99.06 69.85) (end 101.6 69.85) (width 1) (layer "B.Cu") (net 2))
 (segment (start 95.25 62.23) (end 93.98 60.96) (width 1) (layer "B.Cu") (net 2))
 (segment (start 134.62 95.25) (end 135.89 96.52) (width 1) (layer "B.Cu") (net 2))
 (segment (start 147.32 96.52) (end 154.94 88.9) (width 1) (layer "B.Cu") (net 2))
 (segment (start 133.35 90.17) (end 134.62 91.44) (width 1) (layer "B.Cu") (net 2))
 (segment (start 104.14 45.72) (end 140.97 45.72) (width 1) (layer "B.Cu") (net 2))
 (segment (start 93.98 81.28) (end 93.98 71.12) (width 1) (layer "F.Cu") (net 47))
 (segment (start 147.32 87.63) (end 151.13 91.44) (width 1) (layer "F.Cu") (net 47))
 (segment (start 95.25 69.85) (end 96.52 69.85) (width 1) (layer "F.Cu") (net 47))
 (segment (start 146.05 48.26) (end 147.32 49.53) (width 1) (layer "F.Cu") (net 47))
 (segment (start 95.25 82.55) (end 93.98 81.28) (width 1) (layer "F.Cu") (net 47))
 (segment (start 101.6 48.26) (end 93.98 55.88) (width 1) (layer "F.Cu") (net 47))
 (segment (start 96.52 82.55) (end 95.25 82.55) (width 1) (layer "F.Cu") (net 47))
 (segment (start 140.97 48.26) (end 146.05 48.26) (width 1) (layer "F.Cu") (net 47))
 (segment (start 93.98 71.12) (end 95.25 69.85) (width 1) (layer "F.Cu") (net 47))
 (segment (start 147.32 49.53) (end 147.32 87.63) (width 1) (layer "F.Cu") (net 47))
 (segment (start 93.98 55.88) (end 93.98 68.58) (width 1) (layer "F.Cu") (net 47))
 (segment (start 93.98 68.58) (end 95.25 69.85) (width 1) (layer "F.Cu") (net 47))
 (segment (start 140.97 48.26) (end 101.6 48.26) (width 1) (layer "F.Cu") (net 47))
 (segment (start 151.13 91.44) (end 156.21 91.44) (width 1) (layer "F.Cu") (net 47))
 (segment (start 87.63 85.09) (end 87.63 87.63) (width 1) (layer "B.Cu") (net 33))
 (segment (start 99.06 77.47) (end 97.79 78.74) (width 0.4) (layer "B.Cu") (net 33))
 (segment (start 91.44 78.74) (end 87.63 82.55) (width 0.4) (layer "B.Cu") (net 33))
 (segment (start 87.63 82.55) (end 87.63 85.09) (width 0.4) (layer "B.Cu") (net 33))
 (segment (start 97.79 78.74) (end 91.44 78.74) (width 0.4) (layer "B.Cu") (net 33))
 (segment (start 85.09 82.55) (end 85.09 85.09) (width 0.4) (layer "B.Cu") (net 35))
 (segment (start 85.09 85.09) (end 85.09 87.63) (width 1) (layer "B.Cu") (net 35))
 (segment (start 90.17 77.47) (end 85.09 82.55) (width 0.4) (layer "B.Cu") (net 35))
 (segment (start 96.52 77.47) (end 90.17 77.47) (width 0.4) (layer "B.Cu") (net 35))
 (segment (start 90.17 85.09) (end 90.17 87.63) (width 1) (layer "B.Cu") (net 31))
 (segment (start 90.17 82.55) (end 90.17 85.09) (width 0.4) (layer "B.Cu") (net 31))
 (segment (start 92.71 80.01) (end 90.17 82.55) (width 0.4) (layer "B.Cu") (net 31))
 (segment (start 96.52 80.01) (end 92.71 80.01) (width 0.4) (layer "B.Cu") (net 31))
 (segment (start 82.55 85.09) (end 82.55 87.63) (width 1) (layer "B.Cu") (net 37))
 (segment (start 80.01 81.28) (end 82.55 83.82) (width 0.4) (layer "B.Cu") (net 37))
 (segment (start 82.55 83.82) (end 82.55 85.09) (width 0.4) (layer "B.Cu") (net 37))
 (segment (start 69.85 81.28) (end 80.01 81.28) (width 0.4) (layer "B.Cu") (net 37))
 (segment (start 68.58 82.55) (end 69.85 81.28) (width 0.4) (layer "B.Cu") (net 37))
 (segment (start 71.12 82.55) (end 78.74 82.55) (width 0.4) (layer "B.Cu") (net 39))
 (segment (start 78.74 82.55) (end 80.01 83.82) (width 0.4) (layer "B.Cu") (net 39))
 (segment (start 80.01 85.09) (end 80.01 87.63) (width 1) (layer "B.Cu") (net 39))
 (segment (start 80.01 83.82) (end 80.01 85.09) (width 0.4) (layer "B.Cu") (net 39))
 (segment (start 92.71 85.09) (end 92.71 87.63) (width 1) (layer "B.Cu") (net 29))
 (segment (start 99.06 80.01) (end 97.79 81.28) (width 0.4) (layer "B.Cu") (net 29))
 (segment (start 97.79 81.28) (end 93.98 81.28) (width 0.4) (layer "B.Cu") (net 29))
 (segment (start 93.98 81.28) (end 92.71 82.55) (width 0.4) (layer "B.Cu") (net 29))
 (segment (start 92.71 82.55) (end 92.71 85.09) (width 0.4) (layer "B.Cu") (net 29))
 (segment (start 114.3 73.66) (end 140.97 73.66) (width 1) (layer "F.Cu") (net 21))
 (segment (start 102.87 85.09) (end 114.3 73.66) (width 1) (layer "F.Cu") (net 21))
 (segment (start 102.87 87.63) (end 102.87 85.09) (width 1) (layer "F.Cu") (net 21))
 (segment (start 149.86 43.18) (end 152.4 45.72) (width 1) (layer "F.Cu") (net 1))
 (segment (start 140.97 43.18) (end 149.86 43.18) (width 1) (layer "F.Cu") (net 1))
 (segment (start 152.4 45.72) (end 152.4 83.82) (width 1) (layer "F.Cu") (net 1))
 (segment (start 154.94 86.36) (end 156.21 86.36) (width 1) (layer "F.Cu") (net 1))
 (segment (start 152.4 83.82) (end 154.94 86.36) (width 1) (layer "F.Cu") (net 1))
 (segment (start 146.05 93.98) (end 153.67 86.36) (width 1) (layer "B.Cu") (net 1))
 (segment (start 134.62 87.63) (end 137.16 90.17) (width 1) (layer "B.Cu") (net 1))
 (segment (start 128.27 87.63) (end 134.62 87.63) (width 1) (layer "B.Cu") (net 1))
 (segment (start 137.16 93.98) (end 146.05 93.98) (width 1) (layer "B.Cu") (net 1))
 (segment (start 137.16 90.17) (end 137.16 93.98) (width 1) (layer "B.Cu") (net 1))
 (segment (start 153.67 86.36) (end 156.21 86.36) (width 1) (layer "B.Cu") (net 1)))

